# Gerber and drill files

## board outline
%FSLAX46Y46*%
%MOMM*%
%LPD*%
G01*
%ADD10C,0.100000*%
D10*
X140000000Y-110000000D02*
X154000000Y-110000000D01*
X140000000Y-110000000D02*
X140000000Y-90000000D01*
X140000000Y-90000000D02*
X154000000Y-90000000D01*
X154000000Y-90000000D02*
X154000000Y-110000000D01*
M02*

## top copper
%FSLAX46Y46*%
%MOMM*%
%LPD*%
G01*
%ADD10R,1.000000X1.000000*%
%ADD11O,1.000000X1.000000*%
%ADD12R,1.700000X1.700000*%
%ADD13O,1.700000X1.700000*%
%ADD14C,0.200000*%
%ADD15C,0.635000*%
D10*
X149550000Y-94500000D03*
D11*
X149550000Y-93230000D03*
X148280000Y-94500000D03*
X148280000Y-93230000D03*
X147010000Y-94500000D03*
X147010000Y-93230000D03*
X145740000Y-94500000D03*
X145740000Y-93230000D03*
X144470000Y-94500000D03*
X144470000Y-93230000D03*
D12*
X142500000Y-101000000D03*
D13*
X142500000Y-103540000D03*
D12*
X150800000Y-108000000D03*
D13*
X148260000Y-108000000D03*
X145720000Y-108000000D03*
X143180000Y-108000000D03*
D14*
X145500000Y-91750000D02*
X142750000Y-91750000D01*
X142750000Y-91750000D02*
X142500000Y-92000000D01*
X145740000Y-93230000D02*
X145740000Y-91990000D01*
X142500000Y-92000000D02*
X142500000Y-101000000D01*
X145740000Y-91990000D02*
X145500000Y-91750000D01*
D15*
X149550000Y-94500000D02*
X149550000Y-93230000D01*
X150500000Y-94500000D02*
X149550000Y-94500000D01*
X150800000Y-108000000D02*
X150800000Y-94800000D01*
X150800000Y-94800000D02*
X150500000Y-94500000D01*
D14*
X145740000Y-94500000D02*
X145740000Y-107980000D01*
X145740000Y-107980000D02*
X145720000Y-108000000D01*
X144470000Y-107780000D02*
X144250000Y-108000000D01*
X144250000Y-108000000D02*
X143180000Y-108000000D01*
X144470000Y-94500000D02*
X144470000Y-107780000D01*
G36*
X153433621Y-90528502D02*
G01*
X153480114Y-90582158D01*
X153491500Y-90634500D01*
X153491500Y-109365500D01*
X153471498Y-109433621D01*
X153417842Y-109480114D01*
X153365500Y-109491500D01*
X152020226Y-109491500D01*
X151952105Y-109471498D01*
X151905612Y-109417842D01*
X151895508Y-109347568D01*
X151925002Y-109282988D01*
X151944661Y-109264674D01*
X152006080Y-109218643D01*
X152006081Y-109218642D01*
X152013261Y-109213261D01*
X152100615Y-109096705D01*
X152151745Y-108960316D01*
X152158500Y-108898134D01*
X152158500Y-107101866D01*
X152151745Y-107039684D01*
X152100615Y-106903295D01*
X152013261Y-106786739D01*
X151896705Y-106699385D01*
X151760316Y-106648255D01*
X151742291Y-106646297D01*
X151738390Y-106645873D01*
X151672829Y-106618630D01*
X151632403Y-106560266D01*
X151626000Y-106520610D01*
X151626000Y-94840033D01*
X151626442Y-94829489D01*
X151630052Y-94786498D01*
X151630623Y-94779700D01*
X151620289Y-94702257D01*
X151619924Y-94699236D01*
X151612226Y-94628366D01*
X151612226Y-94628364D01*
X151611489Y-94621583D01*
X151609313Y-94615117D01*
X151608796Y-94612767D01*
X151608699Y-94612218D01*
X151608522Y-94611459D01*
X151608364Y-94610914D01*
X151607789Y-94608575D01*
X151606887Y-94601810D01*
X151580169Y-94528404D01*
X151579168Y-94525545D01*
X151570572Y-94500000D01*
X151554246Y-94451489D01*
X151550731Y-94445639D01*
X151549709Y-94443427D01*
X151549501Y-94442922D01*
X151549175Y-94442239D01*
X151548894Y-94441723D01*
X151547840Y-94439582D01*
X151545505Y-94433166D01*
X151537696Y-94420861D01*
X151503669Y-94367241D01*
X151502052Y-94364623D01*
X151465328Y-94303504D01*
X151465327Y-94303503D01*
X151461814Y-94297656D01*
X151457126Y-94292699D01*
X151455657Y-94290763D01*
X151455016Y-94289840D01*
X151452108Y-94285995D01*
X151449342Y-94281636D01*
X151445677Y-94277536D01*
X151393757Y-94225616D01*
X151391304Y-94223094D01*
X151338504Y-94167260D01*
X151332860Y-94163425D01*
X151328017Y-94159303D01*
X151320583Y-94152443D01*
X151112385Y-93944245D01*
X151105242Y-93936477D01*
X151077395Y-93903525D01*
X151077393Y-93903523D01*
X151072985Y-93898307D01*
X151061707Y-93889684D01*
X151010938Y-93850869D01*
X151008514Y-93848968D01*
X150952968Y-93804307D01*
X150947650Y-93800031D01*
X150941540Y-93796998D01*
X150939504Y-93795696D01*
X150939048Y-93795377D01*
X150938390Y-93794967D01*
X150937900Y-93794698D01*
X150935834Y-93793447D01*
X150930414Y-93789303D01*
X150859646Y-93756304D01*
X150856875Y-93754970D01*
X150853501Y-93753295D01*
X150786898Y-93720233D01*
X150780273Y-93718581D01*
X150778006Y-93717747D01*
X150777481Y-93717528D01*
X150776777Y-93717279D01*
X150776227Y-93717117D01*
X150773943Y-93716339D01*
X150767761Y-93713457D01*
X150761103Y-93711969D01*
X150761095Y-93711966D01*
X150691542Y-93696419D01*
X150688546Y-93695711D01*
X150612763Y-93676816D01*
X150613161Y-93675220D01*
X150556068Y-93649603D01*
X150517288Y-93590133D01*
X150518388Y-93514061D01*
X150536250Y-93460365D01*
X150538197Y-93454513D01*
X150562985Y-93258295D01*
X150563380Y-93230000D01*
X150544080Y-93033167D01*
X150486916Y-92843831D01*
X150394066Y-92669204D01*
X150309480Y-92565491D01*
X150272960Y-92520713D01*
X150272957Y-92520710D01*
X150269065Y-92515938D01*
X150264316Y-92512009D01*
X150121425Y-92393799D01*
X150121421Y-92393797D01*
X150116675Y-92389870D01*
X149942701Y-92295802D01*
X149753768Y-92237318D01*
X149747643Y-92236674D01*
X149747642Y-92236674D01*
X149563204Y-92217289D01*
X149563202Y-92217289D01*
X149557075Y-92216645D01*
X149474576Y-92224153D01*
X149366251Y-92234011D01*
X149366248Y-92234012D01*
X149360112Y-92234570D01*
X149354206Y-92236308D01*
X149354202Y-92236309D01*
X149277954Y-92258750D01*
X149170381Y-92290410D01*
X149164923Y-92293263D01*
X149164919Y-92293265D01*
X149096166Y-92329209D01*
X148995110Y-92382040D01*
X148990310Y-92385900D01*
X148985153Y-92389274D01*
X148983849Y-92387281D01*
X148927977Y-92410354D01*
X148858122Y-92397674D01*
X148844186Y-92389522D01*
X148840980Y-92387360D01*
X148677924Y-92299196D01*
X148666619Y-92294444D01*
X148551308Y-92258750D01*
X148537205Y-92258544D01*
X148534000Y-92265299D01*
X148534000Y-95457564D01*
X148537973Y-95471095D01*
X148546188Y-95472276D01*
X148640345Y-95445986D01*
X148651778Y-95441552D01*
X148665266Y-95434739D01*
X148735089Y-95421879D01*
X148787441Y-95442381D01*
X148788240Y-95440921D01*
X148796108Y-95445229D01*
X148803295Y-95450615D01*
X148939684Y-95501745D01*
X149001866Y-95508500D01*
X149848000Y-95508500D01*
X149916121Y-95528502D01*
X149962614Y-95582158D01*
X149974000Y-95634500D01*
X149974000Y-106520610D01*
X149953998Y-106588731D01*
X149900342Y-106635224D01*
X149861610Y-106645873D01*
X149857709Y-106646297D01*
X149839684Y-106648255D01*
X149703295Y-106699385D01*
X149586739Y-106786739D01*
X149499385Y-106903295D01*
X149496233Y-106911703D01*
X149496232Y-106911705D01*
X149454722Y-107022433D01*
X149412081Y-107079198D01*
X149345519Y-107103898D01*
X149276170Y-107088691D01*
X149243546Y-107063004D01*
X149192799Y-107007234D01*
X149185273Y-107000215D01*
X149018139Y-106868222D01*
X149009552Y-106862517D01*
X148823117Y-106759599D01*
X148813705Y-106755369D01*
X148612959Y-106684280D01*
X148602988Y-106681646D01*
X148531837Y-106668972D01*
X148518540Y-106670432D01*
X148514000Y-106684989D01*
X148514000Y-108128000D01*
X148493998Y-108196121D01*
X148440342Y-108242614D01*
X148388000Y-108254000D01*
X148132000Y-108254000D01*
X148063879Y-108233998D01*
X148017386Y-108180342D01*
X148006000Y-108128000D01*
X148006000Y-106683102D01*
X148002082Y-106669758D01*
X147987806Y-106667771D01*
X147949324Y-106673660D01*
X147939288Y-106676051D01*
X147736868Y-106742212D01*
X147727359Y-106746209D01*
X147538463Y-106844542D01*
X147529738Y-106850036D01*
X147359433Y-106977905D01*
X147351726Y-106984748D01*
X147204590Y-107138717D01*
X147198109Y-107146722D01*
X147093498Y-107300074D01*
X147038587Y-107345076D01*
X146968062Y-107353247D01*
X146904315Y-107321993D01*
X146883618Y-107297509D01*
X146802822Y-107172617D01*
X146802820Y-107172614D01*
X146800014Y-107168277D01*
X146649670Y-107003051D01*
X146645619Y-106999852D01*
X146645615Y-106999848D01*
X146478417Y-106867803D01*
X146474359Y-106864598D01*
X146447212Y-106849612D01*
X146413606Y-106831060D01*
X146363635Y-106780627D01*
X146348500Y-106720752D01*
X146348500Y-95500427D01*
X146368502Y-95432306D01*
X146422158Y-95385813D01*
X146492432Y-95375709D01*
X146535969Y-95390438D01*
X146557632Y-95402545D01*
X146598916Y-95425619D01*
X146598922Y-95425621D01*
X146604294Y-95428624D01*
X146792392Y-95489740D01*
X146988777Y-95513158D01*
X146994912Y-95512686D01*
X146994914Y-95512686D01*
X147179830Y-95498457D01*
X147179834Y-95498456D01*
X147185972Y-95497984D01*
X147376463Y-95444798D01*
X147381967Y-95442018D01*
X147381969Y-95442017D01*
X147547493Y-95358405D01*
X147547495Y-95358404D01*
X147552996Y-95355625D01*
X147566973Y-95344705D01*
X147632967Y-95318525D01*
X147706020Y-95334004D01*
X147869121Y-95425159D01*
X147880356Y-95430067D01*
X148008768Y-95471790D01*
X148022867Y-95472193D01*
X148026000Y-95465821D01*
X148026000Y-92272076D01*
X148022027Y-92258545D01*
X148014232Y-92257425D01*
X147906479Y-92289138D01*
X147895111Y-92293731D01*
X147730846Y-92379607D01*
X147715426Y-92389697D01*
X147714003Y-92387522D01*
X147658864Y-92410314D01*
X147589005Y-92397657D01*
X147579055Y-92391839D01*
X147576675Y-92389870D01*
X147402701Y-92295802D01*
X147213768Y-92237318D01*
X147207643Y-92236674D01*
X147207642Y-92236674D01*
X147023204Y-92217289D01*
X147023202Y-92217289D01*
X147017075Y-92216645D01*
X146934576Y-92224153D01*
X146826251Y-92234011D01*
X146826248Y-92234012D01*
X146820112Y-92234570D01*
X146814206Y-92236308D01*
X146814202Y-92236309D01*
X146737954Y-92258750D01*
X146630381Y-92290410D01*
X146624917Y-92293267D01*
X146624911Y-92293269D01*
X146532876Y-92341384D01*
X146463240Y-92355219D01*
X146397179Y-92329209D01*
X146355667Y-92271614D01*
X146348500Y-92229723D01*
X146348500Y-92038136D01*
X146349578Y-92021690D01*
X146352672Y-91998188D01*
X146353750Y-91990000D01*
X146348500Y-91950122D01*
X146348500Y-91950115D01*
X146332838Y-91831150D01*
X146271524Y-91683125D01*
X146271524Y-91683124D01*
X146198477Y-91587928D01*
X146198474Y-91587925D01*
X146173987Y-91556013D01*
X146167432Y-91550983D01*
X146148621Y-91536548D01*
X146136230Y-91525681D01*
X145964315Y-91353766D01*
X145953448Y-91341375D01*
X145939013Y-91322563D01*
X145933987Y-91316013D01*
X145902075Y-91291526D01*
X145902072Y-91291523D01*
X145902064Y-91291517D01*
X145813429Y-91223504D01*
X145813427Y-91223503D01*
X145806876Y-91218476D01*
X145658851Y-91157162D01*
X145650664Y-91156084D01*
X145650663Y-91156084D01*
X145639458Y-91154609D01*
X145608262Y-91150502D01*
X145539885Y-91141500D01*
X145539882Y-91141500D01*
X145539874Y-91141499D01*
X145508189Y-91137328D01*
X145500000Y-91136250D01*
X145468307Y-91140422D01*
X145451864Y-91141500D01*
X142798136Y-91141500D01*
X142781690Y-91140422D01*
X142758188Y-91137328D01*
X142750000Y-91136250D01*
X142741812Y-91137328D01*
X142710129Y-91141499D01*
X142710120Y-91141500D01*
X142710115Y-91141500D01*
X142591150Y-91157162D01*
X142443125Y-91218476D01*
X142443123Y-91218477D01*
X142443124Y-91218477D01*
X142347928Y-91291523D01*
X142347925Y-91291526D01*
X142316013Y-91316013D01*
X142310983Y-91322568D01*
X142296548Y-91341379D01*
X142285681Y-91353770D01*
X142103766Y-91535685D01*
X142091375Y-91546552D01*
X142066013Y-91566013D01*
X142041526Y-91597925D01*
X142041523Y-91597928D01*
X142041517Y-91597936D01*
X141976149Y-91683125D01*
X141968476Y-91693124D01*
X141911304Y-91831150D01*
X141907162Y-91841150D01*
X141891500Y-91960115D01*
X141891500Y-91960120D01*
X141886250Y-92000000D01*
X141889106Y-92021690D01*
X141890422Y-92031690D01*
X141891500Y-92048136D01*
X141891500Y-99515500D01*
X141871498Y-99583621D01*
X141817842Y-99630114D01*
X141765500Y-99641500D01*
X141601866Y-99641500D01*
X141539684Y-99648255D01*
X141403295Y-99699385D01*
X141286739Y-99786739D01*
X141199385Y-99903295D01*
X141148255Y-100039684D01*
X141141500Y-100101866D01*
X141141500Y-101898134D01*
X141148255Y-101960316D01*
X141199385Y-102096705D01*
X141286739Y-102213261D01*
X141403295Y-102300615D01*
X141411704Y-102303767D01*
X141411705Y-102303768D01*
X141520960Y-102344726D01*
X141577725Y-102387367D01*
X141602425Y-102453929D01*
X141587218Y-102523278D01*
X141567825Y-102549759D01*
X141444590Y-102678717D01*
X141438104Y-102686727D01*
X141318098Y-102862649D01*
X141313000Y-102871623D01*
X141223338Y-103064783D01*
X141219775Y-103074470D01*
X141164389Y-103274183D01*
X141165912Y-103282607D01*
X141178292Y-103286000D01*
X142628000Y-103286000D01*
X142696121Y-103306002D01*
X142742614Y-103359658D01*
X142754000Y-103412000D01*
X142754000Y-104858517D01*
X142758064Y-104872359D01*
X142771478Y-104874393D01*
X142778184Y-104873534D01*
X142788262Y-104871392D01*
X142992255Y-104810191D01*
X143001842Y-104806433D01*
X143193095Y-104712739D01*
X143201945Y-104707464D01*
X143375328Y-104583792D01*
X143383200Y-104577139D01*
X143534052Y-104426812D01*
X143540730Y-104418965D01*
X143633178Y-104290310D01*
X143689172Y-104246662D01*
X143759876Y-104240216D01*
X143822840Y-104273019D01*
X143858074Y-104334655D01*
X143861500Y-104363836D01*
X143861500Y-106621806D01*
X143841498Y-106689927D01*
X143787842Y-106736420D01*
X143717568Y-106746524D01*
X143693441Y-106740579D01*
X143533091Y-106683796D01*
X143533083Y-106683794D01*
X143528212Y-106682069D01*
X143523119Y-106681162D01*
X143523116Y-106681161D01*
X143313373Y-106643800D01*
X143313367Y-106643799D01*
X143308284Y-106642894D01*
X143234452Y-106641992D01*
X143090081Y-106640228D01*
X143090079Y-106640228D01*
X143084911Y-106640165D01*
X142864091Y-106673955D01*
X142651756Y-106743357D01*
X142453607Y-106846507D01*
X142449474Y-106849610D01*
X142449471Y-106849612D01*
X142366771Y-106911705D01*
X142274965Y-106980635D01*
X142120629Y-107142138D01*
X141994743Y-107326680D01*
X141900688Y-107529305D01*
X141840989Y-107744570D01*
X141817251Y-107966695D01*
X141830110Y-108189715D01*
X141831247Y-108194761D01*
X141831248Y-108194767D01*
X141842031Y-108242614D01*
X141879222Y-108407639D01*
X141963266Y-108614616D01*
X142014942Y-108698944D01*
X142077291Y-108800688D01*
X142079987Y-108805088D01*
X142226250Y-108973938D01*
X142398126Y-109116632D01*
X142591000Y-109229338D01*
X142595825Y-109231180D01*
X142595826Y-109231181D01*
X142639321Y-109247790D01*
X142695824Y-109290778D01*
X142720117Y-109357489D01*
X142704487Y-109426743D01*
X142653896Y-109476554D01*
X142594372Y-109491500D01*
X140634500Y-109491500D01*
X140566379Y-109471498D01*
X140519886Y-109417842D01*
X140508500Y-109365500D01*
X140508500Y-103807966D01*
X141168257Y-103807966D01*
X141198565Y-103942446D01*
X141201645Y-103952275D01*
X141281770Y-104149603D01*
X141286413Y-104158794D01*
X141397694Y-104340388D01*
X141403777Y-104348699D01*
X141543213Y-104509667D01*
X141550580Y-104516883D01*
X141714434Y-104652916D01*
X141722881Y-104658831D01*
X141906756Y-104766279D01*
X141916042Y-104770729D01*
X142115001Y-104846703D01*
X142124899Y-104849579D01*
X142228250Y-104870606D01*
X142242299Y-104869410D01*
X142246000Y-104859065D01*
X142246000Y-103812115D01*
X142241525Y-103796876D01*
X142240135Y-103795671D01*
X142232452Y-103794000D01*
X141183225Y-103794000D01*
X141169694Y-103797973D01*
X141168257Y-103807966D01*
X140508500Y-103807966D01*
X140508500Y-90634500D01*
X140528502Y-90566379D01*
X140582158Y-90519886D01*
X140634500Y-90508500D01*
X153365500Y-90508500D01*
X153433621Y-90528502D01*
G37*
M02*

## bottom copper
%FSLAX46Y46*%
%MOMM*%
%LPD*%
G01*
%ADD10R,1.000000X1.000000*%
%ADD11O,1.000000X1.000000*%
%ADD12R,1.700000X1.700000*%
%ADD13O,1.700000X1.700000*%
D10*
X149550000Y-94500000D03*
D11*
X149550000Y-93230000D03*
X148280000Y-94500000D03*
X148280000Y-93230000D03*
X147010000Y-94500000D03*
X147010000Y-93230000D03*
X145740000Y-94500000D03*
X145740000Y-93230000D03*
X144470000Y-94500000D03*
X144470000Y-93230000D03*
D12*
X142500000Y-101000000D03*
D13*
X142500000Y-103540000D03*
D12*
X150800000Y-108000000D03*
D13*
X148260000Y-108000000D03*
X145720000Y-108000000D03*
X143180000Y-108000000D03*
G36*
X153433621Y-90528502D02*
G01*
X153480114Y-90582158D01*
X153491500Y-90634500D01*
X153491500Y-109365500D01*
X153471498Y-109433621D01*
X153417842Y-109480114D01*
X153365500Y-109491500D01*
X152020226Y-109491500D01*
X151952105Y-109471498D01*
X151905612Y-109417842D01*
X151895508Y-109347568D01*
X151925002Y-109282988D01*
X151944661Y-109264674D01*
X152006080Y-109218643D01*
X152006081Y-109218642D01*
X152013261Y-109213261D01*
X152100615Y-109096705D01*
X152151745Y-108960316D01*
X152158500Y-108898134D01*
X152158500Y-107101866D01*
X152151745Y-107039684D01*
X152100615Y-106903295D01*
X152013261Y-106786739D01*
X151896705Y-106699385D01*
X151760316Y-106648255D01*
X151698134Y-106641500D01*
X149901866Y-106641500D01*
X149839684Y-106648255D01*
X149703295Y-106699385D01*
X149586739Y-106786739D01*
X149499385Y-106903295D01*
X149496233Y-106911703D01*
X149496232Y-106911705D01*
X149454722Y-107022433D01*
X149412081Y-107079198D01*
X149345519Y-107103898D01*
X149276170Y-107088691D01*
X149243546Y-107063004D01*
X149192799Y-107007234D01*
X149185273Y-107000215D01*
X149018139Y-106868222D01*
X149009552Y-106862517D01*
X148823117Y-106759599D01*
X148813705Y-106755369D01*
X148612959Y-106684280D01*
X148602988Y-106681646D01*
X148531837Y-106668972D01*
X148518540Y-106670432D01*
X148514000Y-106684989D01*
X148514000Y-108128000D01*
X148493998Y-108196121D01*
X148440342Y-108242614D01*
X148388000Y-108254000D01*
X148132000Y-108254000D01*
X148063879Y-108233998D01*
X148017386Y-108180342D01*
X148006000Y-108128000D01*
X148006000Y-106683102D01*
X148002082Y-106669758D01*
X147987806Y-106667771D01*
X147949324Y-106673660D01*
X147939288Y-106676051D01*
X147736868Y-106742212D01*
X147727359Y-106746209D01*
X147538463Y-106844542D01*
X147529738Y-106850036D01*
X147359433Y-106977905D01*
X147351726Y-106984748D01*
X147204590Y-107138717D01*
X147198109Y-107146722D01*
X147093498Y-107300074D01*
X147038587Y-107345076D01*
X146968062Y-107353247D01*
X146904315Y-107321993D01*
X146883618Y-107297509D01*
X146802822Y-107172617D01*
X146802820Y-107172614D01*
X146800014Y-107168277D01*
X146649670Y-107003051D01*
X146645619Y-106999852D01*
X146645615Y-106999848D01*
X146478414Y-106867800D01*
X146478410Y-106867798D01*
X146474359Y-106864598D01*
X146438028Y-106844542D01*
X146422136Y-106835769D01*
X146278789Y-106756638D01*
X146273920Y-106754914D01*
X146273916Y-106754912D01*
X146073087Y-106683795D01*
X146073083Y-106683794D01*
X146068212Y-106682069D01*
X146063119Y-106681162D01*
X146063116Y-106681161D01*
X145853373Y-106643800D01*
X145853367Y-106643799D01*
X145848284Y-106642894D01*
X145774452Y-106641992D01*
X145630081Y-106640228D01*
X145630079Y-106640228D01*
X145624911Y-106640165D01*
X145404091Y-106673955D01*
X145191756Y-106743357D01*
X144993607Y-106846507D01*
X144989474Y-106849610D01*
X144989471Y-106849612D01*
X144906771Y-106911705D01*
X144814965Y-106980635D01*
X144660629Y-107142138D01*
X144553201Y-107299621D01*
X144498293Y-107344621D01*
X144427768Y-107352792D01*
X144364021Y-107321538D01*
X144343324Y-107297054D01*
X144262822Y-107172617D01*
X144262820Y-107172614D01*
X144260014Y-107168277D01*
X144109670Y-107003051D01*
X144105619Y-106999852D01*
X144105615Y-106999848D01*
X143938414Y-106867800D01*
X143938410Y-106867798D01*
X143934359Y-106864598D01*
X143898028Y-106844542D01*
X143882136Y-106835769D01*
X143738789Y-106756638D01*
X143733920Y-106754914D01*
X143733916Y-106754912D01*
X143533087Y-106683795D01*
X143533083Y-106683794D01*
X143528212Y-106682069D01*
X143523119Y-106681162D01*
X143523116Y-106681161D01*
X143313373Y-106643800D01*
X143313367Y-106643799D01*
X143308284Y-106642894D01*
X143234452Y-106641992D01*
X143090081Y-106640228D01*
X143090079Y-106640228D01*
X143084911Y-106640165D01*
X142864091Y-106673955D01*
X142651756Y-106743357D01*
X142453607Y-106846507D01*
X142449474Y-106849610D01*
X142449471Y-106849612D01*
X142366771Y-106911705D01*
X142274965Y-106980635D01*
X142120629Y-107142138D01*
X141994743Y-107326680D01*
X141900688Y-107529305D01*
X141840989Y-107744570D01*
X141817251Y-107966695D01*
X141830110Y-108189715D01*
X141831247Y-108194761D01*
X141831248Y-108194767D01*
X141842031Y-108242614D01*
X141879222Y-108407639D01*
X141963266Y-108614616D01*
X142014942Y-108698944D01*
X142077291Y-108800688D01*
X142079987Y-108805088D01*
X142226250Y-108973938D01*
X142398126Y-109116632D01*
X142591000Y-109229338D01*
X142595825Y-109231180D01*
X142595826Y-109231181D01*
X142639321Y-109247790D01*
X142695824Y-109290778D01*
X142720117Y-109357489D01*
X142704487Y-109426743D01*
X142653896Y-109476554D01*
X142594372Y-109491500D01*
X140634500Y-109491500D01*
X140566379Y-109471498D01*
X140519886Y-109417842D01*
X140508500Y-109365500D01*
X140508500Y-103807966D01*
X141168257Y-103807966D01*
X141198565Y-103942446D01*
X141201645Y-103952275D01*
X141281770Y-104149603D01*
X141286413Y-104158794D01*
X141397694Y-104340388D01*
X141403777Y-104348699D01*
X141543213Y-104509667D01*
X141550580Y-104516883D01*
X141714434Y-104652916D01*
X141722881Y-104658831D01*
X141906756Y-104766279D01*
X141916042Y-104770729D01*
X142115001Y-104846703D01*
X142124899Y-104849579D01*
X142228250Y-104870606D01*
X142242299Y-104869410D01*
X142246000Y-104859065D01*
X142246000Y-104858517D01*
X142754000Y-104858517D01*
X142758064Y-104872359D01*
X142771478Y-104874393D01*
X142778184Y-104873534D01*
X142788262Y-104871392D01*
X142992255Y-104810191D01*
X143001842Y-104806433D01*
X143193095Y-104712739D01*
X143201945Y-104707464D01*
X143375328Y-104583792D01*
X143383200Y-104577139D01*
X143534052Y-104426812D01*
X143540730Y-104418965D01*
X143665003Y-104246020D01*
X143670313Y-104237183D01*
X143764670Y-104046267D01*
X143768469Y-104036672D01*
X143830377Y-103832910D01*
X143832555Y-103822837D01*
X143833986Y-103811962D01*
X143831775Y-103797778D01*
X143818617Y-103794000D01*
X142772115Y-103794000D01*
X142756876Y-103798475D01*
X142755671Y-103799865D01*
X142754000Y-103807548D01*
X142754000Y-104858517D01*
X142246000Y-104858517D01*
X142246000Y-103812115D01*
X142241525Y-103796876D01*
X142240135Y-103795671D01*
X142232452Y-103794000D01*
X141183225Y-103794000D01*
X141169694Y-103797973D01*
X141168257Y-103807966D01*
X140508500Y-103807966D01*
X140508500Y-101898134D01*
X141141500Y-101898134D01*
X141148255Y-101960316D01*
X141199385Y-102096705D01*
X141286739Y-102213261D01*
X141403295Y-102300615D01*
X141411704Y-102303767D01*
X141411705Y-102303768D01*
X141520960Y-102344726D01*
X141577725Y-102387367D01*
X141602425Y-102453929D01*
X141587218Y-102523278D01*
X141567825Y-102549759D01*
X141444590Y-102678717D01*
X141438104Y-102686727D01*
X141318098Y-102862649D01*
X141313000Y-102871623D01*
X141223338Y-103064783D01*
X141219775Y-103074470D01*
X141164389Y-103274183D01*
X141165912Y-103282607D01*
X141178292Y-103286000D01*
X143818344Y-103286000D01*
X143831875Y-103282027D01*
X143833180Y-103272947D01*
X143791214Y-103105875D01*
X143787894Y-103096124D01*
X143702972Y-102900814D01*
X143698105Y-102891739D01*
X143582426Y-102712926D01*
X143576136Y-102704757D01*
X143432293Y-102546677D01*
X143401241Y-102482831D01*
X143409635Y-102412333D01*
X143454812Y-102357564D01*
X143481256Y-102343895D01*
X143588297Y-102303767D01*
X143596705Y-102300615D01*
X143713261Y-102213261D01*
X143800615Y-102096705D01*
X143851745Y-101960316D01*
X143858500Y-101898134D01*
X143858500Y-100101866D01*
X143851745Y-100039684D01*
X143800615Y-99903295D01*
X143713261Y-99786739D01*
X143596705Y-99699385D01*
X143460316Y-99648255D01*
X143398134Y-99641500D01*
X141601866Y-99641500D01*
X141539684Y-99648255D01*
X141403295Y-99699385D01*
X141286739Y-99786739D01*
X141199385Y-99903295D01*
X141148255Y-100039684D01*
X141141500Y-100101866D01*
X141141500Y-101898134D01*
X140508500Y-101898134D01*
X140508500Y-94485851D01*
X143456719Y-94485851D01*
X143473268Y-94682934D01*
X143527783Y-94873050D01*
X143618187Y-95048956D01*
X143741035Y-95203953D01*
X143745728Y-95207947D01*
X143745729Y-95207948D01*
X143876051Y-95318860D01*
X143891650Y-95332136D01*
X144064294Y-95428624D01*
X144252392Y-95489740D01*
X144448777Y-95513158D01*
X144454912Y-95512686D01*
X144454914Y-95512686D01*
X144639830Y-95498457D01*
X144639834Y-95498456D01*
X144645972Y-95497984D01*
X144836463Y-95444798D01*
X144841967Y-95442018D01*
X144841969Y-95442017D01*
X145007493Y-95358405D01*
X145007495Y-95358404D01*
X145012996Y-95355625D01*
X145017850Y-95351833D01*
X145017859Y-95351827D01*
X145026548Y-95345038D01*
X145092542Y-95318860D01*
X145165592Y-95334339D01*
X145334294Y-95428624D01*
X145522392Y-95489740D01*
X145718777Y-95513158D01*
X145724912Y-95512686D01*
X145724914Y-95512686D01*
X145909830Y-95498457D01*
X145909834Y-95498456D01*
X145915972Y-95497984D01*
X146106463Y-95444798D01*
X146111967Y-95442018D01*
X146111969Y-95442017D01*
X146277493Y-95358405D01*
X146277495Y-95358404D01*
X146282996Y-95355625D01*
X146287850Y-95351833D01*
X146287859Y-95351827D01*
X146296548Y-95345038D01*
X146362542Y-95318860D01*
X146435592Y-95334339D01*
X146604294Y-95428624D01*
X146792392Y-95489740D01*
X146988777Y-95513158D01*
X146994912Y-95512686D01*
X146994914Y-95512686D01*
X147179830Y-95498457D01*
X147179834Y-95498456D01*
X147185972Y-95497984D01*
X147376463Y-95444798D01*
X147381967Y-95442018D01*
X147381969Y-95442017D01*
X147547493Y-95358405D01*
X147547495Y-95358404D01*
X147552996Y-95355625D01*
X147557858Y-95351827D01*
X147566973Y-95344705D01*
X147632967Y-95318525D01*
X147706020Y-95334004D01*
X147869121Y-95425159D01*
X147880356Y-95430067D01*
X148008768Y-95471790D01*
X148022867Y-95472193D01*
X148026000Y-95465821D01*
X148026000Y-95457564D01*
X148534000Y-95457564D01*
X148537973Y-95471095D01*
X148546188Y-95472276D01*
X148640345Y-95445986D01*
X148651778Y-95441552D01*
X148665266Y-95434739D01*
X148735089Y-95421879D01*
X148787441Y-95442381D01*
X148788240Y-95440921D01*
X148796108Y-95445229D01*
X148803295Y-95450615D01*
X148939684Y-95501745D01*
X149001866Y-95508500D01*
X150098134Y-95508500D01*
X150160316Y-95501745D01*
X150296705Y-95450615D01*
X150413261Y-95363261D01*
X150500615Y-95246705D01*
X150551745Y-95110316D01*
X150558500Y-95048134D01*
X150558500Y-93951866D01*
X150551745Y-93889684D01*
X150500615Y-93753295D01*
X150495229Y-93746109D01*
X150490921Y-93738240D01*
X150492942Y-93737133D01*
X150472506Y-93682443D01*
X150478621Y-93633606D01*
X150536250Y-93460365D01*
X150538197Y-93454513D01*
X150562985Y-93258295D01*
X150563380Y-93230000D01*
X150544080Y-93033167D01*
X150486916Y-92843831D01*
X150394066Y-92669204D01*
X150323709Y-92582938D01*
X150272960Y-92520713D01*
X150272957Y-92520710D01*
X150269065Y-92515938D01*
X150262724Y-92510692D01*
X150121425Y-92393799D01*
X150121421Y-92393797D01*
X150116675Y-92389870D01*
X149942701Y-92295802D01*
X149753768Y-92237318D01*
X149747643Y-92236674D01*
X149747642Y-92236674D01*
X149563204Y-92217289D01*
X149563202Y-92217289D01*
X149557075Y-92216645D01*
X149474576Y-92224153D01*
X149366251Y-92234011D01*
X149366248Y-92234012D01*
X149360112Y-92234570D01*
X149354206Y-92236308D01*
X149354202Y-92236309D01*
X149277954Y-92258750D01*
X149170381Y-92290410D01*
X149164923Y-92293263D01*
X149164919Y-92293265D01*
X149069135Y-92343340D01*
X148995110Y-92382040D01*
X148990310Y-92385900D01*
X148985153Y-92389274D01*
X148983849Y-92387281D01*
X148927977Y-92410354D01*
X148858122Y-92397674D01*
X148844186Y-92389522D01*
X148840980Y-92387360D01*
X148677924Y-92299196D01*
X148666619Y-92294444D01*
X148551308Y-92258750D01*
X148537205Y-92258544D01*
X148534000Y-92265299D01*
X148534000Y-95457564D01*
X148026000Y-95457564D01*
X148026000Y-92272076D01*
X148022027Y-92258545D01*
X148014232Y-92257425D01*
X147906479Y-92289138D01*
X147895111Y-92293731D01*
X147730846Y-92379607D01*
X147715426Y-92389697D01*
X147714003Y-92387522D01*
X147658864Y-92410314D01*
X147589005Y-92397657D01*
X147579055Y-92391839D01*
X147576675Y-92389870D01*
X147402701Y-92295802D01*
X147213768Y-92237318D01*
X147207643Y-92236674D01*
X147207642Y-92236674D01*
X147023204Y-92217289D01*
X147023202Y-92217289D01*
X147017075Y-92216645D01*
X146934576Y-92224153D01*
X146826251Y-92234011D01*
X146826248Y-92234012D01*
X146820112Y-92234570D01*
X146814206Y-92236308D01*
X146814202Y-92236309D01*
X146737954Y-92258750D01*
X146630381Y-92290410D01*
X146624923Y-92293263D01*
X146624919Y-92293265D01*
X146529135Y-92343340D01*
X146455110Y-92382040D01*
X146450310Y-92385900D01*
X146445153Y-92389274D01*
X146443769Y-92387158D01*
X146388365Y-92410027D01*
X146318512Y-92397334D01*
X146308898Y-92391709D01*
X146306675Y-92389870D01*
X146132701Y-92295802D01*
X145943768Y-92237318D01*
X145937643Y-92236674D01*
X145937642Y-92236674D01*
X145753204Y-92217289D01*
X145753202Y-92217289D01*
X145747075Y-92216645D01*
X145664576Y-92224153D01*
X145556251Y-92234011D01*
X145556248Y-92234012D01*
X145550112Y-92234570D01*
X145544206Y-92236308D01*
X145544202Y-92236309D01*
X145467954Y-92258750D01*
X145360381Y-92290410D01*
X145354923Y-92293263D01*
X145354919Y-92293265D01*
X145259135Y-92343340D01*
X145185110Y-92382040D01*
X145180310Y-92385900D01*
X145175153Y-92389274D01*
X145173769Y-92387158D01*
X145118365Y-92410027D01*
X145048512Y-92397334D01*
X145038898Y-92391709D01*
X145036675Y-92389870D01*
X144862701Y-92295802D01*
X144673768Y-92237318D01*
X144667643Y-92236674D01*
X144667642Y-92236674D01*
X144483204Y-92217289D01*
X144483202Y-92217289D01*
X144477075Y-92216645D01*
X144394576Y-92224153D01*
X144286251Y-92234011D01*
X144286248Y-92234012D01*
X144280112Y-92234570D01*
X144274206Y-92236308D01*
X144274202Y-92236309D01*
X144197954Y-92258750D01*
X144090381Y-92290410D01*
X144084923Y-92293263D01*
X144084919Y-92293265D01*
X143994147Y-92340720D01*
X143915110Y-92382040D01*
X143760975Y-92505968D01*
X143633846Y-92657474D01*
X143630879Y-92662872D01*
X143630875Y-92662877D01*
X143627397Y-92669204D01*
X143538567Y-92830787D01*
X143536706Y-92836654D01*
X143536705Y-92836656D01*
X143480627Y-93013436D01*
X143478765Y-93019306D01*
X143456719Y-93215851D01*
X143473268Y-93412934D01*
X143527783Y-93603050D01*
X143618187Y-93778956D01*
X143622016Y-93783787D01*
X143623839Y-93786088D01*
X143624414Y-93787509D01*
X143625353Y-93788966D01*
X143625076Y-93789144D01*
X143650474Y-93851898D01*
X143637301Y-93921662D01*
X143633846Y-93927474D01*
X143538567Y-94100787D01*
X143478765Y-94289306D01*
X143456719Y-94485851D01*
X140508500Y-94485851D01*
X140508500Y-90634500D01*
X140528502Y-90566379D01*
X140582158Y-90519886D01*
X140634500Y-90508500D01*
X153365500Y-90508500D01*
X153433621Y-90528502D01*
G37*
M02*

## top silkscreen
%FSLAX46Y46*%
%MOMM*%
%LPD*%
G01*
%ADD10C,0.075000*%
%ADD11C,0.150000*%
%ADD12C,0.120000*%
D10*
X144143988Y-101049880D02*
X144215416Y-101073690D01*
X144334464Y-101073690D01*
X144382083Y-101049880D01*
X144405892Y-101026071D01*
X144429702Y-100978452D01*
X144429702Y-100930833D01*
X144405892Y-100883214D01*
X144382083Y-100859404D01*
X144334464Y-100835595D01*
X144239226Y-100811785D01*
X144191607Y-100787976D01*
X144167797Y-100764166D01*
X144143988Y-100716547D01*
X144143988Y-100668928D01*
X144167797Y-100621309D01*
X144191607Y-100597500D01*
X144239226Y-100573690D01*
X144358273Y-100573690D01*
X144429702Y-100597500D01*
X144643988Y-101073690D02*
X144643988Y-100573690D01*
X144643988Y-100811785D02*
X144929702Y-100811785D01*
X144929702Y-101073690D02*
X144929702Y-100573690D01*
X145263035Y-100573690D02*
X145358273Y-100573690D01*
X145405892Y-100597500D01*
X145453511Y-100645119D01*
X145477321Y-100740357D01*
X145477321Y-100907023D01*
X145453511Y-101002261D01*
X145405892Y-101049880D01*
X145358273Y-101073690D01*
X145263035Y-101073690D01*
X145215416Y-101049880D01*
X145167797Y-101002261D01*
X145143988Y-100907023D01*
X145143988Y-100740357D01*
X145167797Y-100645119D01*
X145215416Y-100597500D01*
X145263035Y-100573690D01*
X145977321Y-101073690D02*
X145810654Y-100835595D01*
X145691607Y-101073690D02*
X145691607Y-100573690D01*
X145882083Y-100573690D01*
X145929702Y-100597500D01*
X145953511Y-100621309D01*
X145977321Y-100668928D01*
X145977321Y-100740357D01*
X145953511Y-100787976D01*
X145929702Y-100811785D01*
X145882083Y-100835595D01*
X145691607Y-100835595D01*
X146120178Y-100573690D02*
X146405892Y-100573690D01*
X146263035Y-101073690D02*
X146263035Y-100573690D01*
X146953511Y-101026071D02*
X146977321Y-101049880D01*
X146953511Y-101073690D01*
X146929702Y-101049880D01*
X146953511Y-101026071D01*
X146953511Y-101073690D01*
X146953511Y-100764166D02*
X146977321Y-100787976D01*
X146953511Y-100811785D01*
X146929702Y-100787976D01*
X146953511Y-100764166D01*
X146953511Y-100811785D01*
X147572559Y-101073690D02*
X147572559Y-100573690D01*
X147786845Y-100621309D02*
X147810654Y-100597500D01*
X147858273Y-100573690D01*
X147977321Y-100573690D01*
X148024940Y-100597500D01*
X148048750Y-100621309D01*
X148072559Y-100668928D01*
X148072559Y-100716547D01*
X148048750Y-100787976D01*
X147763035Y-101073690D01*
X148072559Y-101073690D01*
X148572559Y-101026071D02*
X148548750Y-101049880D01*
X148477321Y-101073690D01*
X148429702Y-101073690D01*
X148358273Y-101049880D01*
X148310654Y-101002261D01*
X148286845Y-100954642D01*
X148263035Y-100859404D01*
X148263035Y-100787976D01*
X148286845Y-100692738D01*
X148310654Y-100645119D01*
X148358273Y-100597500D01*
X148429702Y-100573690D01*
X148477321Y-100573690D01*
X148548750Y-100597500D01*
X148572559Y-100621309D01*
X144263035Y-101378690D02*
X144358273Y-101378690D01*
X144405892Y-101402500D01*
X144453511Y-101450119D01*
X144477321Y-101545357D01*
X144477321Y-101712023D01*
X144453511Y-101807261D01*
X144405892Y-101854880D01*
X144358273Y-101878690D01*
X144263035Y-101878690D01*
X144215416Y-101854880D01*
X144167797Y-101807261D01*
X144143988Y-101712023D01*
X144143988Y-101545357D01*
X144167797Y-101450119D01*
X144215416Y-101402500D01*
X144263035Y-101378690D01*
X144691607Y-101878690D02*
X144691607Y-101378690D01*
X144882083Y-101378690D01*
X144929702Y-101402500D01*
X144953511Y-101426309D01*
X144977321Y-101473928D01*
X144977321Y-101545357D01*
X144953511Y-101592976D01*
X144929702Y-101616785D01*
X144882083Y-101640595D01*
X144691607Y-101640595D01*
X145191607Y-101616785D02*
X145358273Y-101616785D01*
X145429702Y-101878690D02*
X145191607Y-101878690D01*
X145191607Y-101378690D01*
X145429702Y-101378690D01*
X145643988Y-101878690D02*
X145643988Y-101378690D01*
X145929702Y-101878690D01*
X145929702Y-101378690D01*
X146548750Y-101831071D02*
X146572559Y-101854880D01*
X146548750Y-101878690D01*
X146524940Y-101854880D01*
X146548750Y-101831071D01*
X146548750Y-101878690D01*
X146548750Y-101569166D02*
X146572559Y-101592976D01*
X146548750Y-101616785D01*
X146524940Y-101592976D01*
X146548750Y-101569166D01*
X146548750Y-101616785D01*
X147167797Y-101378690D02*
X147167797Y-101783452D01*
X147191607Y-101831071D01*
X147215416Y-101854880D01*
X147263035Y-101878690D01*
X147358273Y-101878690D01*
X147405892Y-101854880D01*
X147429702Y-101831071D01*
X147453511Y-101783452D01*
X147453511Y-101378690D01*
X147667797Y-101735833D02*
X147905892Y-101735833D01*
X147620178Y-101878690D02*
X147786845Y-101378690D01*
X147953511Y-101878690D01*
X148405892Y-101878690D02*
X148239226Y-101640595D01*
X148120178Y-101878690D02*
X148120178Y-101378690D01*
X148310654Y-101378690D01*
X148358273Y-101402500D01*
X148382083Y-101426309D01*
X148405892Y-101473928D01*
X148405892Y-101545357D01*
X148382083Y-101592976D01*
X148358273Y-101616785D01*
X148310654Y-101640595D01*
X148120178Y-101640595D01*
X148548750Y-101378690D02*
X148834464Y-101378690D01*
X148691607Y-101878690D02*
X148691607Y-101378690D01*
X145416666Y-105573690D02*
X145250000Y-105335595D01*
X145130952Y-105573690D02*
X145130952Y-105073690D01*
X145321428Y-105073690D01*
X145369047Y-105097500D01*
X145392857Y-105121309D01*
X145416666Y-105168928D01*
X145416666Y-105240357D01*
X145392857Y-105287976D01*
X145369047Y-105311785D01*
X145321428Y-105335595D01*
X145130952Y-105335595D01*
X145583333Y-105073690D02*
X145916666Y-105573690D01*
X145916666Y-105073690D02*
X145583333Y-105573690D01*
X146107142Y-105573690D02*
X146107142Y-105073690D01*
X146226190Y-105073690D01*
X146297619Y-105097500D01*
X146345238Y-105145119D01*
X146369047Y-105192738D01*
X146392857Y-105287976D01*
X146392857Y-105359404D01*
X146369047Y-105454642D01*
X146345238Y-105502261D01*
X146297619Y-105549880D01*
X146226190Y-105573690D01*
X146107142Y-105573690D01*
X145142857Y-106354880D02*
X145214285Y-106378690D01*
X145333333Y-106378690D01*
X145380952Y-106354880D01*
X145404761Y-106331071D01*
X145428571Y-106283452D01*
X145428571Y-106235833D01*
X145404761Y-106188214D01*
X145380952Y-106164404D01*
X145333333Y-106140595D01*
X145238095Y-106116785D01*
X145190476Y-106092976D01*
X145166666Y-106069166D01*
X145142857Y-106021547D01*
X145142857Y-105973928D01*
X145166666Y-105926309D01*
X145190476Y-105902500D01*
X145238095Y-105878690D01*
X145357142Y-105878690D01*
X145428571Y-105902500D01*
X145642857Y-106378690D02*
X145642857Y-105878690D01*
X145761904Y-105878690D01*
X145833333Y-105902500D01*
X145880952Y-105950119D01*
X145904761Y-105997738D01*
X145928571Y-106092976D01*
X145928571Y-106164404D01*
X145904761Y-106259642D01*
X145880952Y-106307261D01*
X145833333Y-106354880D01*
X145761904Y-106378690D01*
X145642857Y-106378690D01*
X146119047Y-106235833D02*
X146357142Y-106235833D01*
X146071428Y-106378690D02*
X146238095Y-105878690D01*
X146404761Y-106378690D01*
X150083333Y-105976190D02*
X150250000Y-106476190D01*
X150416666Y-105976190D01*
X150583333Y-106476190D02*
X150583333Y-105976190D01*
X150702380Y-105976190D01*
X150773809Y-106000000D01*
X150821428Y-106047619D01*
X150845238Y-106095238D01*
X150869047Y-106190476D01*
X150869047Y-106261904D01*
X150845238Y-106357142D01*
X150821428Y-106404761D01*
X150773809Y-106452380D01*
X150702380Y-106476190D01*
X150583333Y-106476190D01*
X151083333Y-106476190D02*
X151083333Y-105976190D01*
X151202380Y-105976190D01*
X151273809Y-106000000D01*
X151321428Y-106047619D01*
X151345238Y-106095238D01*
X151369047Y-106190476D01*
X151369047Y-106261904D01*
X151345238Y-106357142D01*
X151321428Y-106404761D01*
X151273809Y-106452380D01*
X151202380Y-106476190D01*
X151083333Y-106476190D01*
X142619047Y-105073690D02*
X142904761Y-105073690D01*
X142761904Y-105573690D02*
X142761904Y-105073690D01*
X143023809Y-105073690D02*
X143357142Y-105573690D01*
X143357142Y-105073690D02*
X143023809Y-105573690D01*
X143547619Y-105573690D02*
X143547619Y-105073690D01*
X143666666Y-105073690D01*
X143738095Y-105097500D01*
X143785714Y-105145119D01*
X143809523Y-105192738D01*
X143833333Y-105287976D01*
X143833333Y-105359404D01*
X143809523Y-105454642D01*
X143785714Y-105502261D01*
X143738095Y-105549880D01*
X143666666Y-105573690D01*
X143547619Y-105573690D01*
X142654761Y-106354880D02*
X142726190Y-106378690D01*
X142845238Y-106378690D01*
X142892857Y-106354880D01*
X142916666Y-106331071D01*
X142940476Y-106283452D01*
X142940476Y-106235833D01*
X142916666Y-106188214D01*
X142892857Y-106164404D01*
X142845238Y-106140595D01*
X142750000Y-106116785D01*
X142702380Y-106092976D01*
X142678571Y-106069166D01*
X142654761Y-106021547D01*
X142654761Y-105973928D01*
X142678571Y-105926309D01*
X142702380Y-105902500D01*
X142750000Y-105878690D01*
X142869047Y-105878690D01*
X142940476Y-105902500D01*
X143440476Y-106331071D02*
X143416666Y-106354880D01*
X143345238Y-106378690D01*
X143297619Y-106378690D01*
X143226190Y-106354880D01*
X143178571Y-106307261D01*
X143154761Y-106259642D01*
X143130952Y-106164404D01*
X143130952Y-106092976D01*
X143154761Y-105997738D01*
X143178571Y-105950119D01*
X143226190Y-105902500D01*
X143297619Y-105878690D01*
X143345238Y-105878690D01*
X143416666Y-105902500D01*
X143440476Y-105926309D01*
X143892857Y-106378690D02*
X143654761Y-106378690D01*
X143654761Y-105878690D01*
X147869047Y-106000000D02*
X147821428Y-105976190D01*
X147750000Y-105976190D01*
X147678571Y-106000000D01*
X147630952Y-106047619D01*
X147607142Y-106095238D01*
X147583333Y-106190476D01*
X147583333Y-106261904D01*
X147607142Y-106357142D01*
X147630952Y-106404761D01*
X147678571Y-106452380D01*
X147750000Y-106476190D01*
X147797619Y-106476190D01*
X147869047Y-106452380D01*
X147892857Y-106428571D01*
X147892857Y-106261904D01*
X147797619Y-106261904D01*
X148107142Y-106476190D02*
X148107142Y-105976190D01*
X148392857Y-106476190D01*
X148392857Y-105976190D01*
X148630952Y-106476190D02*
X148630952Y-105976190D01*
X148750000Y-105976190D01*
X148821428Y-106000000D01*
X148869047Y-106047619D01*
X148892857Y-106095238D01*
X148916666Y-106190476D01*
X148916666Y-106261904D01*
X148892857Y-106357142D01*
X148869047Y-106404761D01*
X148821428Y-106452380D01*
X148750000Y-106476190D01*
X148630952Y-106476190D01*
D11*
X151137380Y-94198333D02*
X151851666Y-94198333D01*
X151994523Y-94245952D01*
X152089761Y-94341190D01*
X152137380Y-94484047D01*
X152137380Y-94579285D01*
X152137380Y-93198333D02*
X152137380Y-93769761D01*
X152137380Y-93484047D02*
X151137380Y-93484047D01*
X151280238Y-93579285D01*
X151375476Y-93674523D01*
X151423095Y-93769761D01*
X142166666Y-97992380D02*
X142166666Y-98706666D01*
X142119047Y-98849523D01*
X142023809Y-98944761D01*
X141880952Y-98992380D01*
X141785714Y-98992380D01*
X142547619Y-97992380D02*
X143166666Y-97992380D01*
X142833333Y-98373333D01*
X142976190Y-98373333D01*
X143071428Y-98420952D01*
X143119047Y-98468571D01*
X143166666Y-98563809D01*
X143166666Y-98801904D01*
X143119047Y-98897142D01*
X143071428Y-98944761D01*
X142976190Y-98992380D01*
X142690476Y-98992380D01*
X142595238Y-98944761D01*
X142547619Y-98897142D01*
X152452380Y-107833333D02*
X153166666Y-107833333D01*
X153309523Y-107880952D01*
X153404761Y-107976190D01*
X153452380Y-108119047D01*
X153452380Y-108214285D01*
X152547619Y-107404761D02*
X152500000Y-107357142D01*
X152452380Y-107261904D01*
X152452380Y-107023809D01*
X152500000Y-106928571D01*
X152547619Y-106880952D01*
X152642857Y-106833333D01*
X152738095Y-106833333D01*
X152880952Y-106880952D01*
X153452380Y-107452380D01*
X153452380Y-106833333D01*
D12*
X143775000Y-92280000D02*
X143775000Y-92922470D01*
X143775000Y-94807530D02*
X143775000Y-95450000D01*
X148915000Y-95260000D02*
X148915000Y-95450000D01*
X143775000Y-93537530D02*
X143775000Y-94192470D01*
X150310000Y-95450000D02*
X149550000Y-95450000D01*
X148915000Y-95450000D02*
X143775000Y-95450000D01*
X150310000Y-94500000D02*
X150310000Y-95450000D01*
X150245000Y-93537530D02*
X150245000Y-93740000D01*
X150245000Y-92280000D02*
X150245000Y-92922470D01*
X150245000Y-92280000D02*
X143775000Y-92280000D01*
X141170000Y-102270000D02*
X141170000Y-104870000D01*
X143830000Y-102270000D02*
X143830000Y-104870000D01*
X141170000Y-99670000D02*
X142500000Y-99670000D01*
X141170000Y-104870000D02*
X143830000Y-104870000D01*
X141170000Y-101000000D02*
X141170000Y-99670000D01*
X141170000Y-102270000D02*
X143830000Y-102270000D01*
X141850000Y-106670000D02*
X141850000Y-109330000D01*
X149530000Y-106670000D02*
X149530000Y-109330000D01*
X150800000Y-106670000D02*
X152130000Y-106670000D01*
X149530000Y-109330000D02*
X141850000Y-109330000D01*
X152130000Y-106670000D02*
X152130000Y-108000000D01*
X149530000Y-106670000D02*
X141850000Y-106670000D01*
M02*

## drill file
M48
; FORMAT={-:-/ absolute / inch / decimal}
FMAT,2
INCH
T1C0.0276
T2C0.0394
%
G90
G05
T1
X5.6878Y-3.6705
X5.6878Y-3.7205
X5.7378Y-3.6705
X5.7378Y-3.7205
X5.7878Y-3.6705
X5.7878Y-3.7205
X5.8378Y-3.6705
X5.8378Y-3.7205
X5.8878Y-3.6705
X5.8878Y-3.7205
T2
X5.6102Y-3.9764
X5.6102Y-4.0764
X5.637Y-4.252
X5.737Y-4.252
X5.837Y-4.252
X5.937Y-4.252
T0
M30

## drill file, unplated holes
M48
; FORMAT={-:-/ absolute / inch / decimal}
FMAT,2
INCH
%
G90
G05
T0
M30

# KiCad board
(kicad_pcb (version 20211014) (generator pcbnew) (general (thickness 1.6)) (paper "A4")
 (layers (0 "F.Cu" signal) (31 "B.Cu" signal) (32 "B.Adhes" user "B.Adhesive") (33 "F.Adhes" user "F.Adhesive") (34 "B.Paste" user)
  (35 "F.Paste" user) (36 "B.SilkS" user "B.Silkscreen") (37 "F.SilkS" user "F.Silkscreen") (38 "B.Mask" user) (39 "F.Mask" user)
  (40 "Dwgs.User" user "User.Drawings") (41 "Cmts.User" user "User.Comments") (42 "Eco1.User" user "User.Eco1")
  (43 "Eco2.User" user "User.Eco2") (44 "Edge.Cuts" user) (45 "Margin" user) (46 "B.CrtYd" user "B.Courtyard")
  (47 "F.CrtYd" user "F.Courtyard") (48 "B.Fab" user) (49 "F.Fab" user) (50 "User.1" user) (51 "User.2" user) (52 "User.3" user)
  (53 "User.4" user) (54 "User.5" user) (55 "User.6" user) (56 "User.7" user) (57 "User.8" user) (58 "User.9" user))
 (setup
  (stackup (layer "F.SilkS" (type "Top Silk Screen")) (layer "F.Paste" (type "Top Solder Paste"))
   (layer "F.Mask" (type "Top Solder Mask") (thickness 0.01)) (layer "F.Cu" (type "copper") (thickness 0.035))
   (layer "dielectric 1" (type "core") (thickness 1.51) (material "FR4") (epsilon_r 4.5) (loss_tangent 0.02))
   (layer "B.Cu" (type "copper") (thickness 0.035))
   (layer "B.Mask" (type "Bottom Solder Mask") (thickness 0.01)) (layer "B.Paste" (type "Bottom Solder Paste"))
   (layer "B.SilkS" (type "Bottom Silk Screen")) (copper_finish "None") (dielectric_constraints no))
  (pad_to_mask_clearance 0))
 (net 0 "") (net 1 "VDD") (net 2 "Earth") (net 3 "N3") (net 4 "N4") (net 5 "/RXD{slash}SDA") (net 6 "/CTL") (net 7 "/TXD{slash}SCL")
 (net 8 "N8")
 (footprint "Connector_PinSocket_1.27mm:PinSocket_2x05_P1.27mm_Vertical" (layer "F.Cu") (at 149.55 94.5 -90)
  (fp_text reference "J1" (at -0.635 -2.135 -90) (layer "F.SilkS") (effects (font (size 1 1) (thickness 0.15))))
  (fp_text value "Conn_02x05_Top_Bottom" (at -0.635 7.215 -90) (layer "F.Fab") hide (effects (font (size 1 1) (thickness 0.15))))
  (fp_line (start -2.22 5.775) (end -1.57753 5.775) (layer "F.SilkS") (width 0.12))
  (fp_line (start 0.30753 5.775) (end 0.95 5.775) (layer "F.SilkS") (width 0.12))
  (fp_line (start 0.76 0.635) (end 0.95 0.635) (layer "F.SilkS") (width 0.12))
  (fp_line (start -0.96247 5.775) (end -0.30753 5.775) (layer "F.SilkS") (width 0.12))
  (fp_line (start 0.95 -0.76) (end 0.95 0) (layer "F.SilkS") (width 0.12))
  (fp_line (start 0.95 0.635) (end 0.95 5.775) (layer "F.SilkS") (width 0.12))
  (fp_line (start 0 -0.76) (end 0.95 -0.76) (layer "F.SilkS") (width 0.12))
  (fp_line (start -0.96247 -0.695) (end -0.76 -0.695) (layer "F.SilkS") (width 0.12))
  (fp_line (start -2.22 -0.695) (end -1.57753 -0.695) (layer "F.SilkS") (width 0.12))
  (fp_line (start -2.22 -0.695) (end -2.22 5.775) (layer "F.SilkS") (width 0.12))
  (pad "1" thru_hole rect (at 0 0 270) (size 1 1) (drill 0.7) (layers *.Cu *.Mask) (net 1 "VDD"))
  (pad "2" thru_hole oval (at -1.27 0 270) (size 1 1) (drill 0.7) (layers *.Cu *.Mask) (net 1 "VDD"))
  (pad "3" thru_hole oval (at 0 1.27 270) (size 1 1) (drill 0.7) (layers *.Cu *.Mask) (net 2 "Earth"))
  (pad "4" thru_hole oval (at -1.27 1.27 270) (size 1 1) (drill 0.7) (layers *.Cu *.Mask) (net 2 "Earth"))
  (pad "5" thru_hole oval (at 0 2.54 270) (size 1 1) (drill 0.7) (layers *.Cu *.Mask) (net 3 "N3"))
  (pad "6" thru_hole oval (at -1.27 2.54 270) (size 1 1) (drill 0.7) (layers *.Cu *.Mask) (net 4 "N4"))
  (pad "7" thru_hole oval (at 0 3.81 270) (size 1 1) (drill 0.7) (layers *.Cu *.Mask) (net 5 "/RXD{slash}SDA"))
  (pad "8" thru_hole oval (at -1.27 3.81 270) (size 1 1) (drill 0.7) (layers *.Cu *.Mask) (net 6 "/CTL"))
  (pad "9" thru_hole oval (at 0 5.08 270) (size 1 1) (drill 0.7) (layers *.Cu *.Mask) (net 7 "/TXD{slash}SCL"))
  (pad "10" thru_hole oval (at -1.27 5.08 270) (size 1 1) (drill 0.7) (layers *.Cu *.Mask) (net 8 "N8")))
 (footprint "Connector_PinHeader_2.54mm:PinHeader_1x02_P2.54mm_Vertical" (layer "F.Cu") (at 142.5 101)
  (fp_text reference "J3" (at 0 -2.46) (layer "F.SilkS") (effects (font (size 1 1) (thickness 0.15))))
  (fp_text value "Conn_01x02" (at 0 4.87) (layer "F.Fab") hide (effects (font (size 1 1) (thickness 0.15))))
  (fp_line (start -1.33 1.27) (end -1.33 3.87) (layer "F.SilkS") (width 0.12))
  (fp_line (start 1.33 1.27) (end 1.33 3.87) (layer "F.SilkS") (width 0.12))
  (fp_line (start -1.33 -1.33) (end 0 -1.33) (layer "F.SilkS") (width 0.12))
  (fp_line (start -1.33 3.87) (end 1.33 3.87) (layer "F.SilkS") (width 0.12))
  (fp_line (start -1.33 0) (end -1.33 -1.33) (layer "F.SilkS") (width 0.12))
  (fp_line (start -1.33 1.27) (end 1.33 1.27) (layer "F.SilkS") (width 0.12))
  (pad "1" thru_hole rect (at 0 0) (size 1.7 1.7) (drill 1) (layers *.Cu *.Mask) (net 6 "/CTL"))
  (pad "2" thru_hole oval (at 0 2.54) (size 1.7 1.7) (drill 1) (layers *.Cu *.Mask) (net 2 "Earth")))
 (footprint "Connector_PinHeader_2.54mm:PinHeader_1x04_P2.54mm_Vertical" (layer "F.Cu") (at 150.8 108 -90)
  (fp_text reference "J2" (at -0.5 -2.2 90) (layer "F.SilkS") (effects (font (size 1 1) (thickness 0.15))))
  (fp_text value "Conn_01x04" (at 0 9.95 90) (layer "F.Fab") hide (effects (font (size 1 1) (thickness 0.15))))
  (fp_line (start -1.33 8.95) (end 1.33 8.95) (layer "F.SilkS") (width 0.12))
  (fp_line (start -1.33 1.27) (end 1.33 1.27) (layer "F.SilkS") (width 0.12))
  (fp_line (start -1.33 0) (end -1.33 -1.33) (layer "F.SilkS") (width 0.12))
  (fp_line (start 1.33 1.27) (end 1.33 8.95) (layer "F.SilkS") (width 0.12))
  (fp_line (start -1.33 -1.33) (end 0 -1.33) (layer "F.SilkS") (width 0.12))
  (fp_line (start -1.33 1.27) (end -1.33 8.95) (layer "F.SilkS") (width 0.12))
  (pad "1" thru_hole rect (at 0 0 270) (size 1.7 1.7) (drill 1) (layers *.Cu *.Mask) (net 1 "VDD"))
  (pad "2" thru_hole oval (at 0 2.54 270) (size 1.7 1.7) (drill 1) (layers *.Cu *.Mask) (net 2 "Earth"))
  (pad "3" thru_hole oval (at 0 5.08 270) (size 1.7 1.7) (drill 1) (layers *.Cu *.Mask) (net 5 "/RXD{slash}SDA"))
  (pad "4" thru_hole oval (at 0 7.62 270) (size 1.7 1.7) (drill 1) (layers *.Cu *.Mask) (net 7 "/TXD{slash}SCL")))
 (gr_line (start 140 110) (end 154 110) (layer "Edge.Cuts") (width 0.1))
 (gr_line (start 140 110) (end 140 90) (layer "Edge.Cuts") (width 0.1))
 (gr_line (start 140 90) (end 154 90) (layer "Edge.Cuts") (width 0.1))
 (gr_line (start 154 90) (end 154 110) (layer "Edge.Cuts") (width 0.1))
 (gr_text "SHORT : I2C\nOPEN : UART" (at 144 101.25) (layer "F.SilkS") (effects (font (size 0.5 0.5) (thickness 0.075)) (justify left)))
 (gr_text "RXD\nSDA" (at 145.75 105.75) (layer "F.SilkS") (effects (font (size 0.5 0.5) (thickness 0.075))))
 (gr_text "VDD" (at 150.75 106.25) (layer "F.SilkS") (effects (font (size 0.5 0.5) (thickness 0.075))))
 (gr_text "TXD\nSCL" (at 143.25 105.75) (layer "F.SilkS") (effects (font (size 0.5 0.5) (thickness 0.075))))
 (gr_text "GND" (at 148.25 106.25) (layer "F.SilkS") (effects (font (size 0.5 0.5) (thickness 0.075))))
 (segment (start 149.55 94.5) (end 149.55 93.23) (width 0.635) (layer "F.Cu") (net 1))
 (segment (start 150.5 94.5) (end 149.55 94.5) (width 0.635) (layer "F.Cu") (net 1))
 (segment (start 150.8 108) (end 150.8 94.8) (width 0.635) (layer "F.Cu") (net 1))
 (segment (start 150.8 94.8) (end 150.5 94.5) (width 0.635) (layer "F.Cu") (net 1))
 (segment (start 145.74 94.5) (end 145.74 107.98) (width 0.2) (layer "F.Cu") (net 5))
 (segment (start 145.74 107.98) (end 145.72 108) (width 0.2) (layer "F.Cu") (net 5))
 (segment (start 145.74 91.99) (end 145.5 91.75) (width 0.2) (layer "F.Cu") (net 6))
 (segment (start 142.5 92) (end 142.5 101) (width 0.2) (layer "F.Cu") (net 6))
 (segment (start 145.5 91.75) (end 142.75 91.75) (width 0.2) (layer "F.Cu") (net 6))
 (segment (start 142.75 91.75) (end 142.5 92) (width 0.2) (layer "F.Cu") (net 6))
 (segment (start 145.74 93.23) (end 145.74 91.99) (width 0.2) (layer "F.Cu") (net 6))
 (segment (start 144.47 107.78) (end 144.25 108) (width 0.2) (layer "F.Cu") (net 7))
 (segment (start 144.25 108) (end 143.18 108) (width 0.2) (layer "F.Cu") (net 7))
 (segment (start 144.47 94.5) (end 144.47 107.78) (width 0.2) (layer "F.Cu") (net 7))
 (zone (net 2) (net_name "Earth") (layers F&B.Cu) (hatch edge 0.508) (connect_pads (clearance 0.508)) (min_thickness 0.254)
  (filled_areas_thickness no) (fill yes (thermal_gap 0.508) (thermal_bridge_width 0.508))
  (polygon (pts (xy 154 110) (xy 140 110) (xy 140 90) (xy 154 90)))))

